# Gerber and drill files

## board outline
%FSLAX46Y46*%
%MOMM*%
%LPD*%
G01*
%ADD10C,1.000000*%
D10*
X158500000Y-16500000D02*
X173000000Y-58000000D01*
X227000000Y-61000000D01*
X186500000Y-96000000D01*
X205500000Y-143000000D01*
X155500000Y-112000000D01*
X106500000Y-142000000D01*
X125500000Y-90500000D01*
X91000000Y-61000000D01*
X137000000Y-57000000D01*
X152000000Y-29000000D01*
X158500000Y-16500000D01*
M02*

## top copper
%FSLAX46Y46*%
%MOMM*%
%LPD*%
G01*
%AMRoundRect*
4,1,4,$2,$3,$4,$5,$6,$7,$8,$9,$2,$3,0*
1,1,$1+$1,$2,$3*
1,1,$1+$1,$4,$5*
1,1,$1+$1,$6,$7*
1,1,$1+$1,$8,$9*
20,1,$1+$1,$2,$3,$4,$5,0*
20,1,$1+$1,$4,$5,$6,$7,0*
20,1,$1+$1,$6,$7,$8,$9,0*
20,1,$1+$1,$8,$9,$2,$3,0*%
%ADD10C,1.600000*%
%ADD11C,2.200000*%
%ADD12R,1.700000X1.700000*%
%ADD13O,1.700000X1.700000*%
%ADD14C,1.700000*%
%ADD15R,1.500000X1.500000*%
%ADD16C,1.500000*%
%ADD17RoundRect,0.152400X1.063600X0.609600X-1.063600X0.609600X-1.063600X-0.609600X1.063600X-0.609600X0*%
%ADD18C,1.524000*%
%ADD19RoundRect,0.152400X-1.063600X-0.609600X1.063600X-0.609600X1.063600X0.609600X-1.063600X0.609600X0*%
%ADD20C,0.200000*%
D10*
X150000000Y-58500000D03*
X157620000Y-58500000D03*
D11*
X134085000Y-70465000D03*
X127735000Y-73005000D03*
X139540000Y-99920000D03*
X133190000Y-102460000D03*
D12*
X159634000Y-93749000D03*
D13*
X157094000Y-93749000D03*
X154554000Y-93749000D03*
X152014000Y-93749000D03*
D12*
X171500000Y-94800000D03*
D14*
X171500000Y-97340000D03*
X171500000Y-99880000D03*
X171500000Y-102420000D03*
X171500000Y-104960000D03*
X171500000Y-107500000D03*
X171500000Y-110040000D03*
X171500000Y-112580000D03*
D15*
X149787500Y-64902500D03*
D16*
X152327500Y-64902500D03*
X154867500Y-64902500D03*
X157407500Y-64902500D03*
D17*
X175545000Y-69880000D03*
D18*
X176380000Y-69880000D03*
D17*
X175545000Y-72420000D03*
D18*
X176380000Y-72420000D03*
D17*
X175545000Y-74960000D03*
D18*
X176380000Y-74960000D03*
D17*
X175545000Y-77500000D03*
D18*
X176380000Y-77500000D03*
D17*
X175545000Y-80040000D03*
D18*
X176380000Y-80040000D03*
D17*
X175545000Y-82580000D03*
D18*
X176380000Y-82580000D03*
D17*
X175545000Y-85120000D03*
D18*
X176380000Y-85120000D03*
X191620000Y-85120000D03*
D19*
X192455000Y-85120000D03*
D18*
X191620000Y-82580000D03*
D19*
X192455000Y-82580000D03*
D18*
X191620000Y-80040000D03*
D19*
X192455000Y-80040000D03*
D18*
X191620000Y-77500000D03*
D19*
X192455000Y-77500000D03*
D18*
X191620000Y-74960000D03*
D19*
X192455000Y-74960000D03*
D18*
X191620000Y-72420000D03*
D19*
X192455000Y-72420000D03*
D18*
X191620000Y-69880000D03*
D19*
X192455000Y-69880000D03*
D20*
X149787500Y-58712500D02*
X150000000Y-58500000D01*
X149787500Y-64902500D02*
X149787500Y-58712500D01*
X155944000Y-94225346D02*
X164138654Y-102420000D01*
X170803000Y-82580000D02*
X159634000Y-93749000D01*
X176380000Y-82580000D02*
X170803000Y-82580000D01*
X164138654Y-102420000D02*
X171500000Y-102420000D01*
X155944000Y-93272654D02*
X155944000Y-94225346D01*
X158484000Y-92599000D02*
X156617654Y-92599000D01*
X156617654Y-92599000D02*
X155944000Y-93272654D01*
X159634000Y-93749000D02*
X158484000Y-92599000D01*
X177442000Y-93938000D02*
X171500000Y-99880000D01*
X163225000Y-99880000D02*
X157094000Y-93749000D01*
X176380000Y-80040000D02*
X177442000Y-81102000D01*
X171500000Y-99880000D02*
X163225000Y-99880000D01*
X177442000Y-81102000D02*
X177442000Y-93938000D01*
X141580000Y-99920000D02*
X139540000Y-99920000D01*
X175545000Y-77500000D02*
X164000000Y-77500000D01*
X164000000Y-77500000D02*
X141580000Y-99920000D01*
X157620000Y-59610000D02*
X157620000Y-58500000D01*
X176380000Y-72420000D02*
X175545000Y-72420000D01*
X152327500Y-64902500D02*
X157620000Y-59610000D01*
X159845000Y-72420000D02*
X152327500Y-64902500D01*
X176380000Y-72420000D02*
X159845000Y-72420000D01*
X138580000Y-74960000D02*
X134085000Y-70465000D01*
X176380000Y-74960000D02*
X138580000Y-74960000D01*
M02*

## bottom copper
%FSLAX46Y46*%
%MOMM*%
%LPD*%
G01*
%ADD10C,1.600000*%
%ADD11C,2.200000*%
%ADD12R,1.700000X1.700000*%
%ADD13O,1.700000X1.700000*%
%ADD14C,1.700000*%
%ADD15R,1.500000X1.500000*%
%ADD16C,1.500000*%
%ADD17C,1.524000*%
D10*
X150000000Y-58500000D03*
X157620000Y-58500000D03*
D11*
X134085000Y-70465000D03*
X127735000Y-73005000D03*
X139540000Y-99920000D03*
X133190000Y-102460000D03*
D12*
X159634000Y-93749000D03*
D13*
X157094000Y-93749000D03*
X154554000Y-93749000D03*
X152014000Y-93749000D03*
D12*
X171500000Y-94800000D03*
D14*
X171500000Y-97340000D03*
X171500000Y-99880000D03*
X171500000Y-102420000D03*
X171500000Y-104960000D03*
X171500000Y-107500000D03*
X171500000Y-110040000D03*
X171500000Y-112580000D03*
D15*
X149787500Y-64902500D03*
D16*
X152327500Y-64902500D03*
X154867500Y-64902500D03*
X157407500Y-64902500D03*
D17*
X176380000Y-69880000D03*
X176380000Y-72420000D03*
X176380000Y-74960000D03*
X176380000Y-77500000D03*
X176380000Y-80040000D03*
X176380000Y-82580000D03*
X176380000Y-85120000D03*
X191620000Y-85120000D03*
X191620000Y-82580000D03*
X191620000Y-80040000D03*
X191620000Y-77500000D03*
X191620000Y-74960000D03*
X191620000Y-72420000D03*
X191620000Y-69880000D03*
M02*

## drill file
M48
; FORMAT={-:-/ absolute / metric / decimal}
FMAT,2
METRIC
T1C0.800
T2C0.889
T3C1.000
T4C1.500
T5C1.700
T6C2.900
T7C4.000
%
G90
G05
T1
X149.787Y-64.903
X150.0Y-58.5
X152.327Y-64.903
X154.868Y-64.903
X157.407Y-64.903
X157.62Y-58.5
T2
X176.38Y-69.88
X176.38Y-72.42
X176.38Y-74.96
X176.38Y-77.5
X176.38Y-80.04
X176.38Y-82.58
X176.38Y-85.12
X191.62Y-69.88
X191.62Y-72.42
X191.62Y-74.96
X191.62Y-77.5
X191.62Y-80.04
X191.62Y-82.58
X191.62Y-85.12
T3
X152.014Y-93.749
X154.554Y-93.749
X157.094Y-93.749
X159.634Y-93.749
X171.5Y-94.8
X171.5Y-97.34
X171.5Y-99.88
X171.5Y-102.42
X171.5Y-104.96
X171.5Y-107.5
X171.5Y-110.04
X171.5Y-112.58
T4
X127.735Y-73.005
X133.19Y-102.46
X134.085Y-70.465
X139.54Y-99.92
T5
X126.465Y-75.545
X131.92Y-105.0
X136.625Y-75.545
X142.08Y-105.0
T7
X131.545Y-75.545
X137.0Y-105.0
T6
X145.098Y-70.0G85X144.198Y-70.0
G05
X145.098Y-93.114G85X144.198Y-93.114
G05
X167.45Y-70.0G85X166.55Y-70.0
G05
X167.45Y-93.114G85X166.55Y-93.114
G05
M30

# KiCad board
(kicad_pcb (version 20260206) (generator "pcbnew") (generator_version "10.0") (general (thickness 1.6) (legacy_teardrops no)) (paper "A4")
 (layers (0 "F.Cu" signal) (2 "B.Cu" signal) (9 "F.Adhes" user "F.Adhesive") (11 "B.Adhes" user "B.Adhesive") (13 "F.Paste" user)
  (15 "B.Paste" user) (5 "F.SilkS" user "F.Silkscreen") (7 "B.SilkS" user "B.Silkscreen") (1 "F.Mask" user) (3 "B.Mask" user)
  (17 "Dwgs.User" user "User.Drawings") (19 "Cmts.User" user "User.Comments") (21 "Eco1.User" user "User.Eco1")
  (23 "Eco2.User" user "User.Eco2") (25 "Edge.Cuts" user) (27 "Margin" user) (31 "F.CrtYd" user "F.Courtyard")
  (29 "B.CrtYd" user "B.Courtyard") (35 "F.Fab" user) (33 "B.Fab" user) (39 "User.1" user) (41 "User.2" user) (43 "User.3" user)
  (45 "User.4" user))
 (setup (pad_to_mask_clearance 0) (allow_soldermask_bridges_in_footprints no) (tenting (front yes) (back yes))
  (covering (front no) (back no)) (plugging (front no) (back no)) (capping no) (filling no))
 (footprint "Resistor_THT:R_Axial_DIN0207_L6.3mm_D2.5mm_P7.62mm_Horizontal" (layer "F.Cu") (at 150 58.5)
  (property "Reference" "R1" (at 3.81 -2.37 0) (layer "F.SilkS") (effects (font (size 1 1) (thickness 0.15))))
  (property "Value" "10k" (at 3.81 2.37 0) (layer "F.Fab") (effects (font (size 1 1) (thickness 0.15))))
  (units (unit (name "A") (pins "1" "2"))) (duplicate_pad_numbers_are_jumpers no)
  (pad "1" thru_hole circle (at 0 0) (size 1.6 1.6) (drill 0.8) (layers "*.Cu" "*.Mask") (remove_unused_layers no) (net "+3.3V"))
  (pad "2" thru_hole circle (at 7.62 0) (size 1.6 1.6) (drill 0.8) (layers "*.Cu" "*.Mask") (remove_unused_layers no) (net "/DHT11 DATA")))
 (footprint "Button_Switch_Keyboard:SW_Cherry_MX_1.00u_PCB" (layer "F.Cu") (at 134.085 70.465)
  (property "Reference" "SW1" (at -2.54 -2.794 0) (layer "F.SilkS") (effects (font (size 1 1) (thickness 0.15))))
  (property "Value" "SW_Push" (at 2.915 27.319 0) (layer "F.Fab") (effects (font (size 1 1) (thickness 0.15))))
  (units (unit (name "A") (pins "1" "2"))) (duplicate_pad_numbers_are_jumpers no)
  (pad "" np_thru_hole circle (at -7.62 5.08) (size 1.7 1.7) (drill 1.7) (layers "*.Cu" "*.Mask"))
  (pad "" np_thru_hole circle (at -2.54 5.08) (size 4 4) (drill 4) (layers "*.Cu" "*.Mask"))
  (pad "" np_thru_hole circle (at 2.54 5.08) (size 1.7 1.7) (drill 1.7) (layers "*.Cu" "*.Mask"))
  (pad "1" thru_hole circle (at 0 0) (size 2.2 2.2) (drill 1.5) (layers "*.Cu" "*.Mask") (remove_unused_layers no) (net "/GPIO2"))
  (pad "2" thru_hole circle (at -6.35 2.54) (size 2.2 2.2) (drill 1.5) (layers "*.Cu" "*.Mask") (remove_unused_layers no) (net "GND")))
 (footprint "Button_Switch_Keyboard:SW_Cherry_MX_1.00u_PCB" (layer "F.Cu") (at 139.54 99.92)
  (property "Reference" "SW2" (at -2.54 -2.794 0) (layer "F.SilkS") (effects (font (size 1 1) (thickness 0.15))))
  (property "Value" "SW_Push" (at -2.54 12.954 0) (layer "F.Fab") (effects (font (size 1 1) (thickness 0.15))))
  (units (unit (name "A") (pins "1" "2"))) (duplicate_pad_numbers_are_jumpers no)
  (pad "" np_thru_hole circle (at -7.62 5.08) (size 1.7 1.7) (drill 1.7) (layers "*.Cu" "*.Mask"))
  (pad "" np_thru_hole circle (at -2.54 5.08) (size 4 4) (drill 4) (layers "*.Cu" "*.Mask"))
  (pad "" np_thru_hole circle (at 2.54 5.08) (size 1.7 1.7) (drill 1.7) (layers "*.Cu" "*.Mask"))
  (pad "1" thru_hole circle (at 0 0) (size 2.2 2.2) (drill 1.5) (layers "*.Cu" "*.Mask") (remove_unused_layers no) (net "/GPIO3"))
  (pad "2" thru_hole circle (at -6.35 2.54) (size 2.2 2.2) (drill 1.5) (layers "*.Cu" "*.Mask") (remove_unused_layers no) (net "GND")))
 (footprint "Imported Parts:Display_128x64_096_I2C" (layer "F.Cu") (at 155.824 93.749 180)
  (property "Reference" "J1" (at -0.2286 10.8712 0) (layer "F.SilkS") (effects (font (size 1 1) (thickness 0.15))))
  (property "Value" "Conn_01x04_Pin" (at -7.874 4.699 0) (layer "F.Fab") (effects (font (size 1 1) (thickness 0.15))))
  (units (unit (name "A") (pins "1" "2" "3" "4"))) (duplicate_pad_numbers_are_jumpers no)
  (pad "" np_thru_hole oval (at -11.176 0.635 180) (size 3.8 2.9) (drill oval 3.8 2.9) (layers "*.Cu" "*.Mask"))
  (pad "" np_thru_hole oval (at -11.176 23.749 180) (size 3.8 2.9) (drill oval 3.8 2.9) (layers "*.Cu" "*.Mask"))
  (pad "" np_thru_hole oval (at 11.176 0.635 180) (size 3.8 2.9) (drill oval 3.8 2.9) (layers "*.Cu" "*.Mask"))
  (pad "" np_thru_hole oval (at 11.176 23.749 180) (size 3.8 2.9) (drill oval 3.8 2.9) (layers "*.Cu" "*.Mask"))
  (pad "1" thru_hole rect (at -3.81 0 270) (size 1.7 1.7) (drill 1) (layers "*.Cu" "*.Mask") (remove_unused_layers no) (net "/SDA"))
  (pad "2" thru_hole oval (at -1.27 0 270) (size 1.7 1.7) (drill 1) (layers "*.Cu" "*.Mask") (remove_unused_layers no) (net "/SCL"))
  (pad "3" thru_hole oval (at 1.27 0 270) (size 1.7 1.7) (drill 1) (layers "*.Cu" "*.Mask") (remove_unused_layers no) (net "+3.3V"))
  (pad "4" thru_hole oval (at 3.81 0 270) (size 1.7 1.7) (drill 1) (layers "*.Cu" "*.Mask") (remove_unused_layers no) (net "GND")))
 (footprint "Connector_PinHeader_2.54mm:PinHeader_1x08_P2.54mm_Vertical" (layer "F.Cu") (at 171.5 94.8)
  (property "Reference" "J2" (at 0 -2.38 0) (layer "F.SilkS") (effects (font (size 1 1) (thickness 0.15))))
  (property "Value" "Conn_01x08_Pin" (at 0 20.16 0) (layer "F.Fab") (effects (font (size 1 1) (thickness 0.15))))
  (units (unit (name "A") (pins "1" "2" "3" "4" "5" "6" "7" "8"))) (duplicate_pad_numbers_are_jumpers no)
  (pad "1" thru_hole rect (at 0 0) (size 1.7 1.7) (drill 1) (layers "*.Cu" "*.Mask") (remove_unused_layers no) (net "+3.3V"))
  (pad "2" thru_hole circle (at 0 2.54) (size 1.7 1.7) (drill 1) (layers "*.Cu" "*.Mask") (remove_unused_layers no) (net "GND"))
  (pad "3" thru_hole circle (at 0 5.08) (size 1.7 1.7) (drill 1) (layers "*.Cu" "*.Mask") (remove_unused_layers no) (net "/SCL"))
  (pad "4" thru_hole circle (at 0 7.62) (size 1.7 1.7) (drill 1) (layers "*.Cu" "*.Mask") (remove_unused_layers no) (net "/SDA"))
  (pad "5" thru_hole circle (at 0 10.16) (size 1.7 1.7) (drill 1) (layers "*.Cu" "*.Mask") (remove_unused_layers no)
   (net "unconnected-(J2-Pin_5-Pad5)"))
  (pad "6" thru_hole circle (at 0 12.7) (size 1.7 1.7) (drill 1) (layers "*.Cu" "*.Mask") (remove_unused_layers no)
   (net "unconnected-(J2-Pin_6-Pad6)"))
  (pad "7" thru_hole circle (at 0 15.24) (size 1.7 1.7) (drill 1) (layers "*.Cu" "*.Mask") (remove_unused_layers no)
   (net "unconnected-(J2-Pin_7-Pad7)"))
  (pad "8" thru_hole circle (at 0 17.78) (size 1.7 1.7) (drill 1) (layers "*.Cu" "*.Mask") (remove_unused_layers no)
   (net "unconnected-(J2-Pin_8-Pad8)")))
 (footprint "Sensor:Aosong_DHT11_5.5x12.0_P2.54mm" (layer "F.Cu") (at 149.7875 64.9025 90)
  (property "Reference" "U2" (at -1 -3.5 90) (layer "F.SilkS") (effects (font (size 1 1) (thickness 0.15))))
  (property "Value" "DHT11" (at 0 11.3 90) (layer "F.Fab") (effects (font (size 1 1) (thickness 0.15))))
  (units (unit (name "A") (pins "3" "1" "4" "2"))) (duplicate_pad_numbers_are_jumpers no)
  (pad "1" thru_hole rect (at 0 0 90) (size 1.5 1.5) (drill 0.8) (layers "*.Cu" "*.Mask") (remove_unused_layers no) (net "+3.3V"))
  (pad "2" thru_hole circle (at 0 2.54 90) (size 1.5 1.5) (drill 0.8) (layers "*.Cu" "*.Mask") (remove_unused_layers no) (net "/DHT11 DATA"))
  (pad "3" thru_hole circle (at 0 5.08 90) (size 1.5 1.5) (drill 0.8) (layers "*.Cu" "*.Mask") (remove_unused_layers no)
   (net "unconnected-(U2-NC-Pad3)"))
  (pad "4" thru_hole circle (at 0 7.62 90) (size 1.5 1.5) (drill 0.8) (layers "*.Cu" "*.Mask") (remove_unused_layers no) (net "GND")))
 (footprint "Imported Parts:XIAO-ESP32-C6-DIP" (layer "F.Cu") (at 184 77.5 90)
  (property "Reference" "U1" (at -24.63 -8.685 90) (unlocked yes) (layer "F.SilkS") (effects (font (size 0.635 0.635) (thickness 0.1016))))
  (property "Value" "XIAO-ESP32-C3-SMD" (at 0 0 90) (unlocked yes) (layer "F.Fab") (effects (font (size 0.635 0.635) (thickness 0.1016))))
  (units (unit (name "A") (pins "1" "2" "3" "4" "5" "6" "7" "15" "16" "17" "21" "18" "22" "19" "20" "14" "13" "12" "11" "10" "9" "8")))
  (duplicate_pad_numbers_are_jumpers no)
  (pad "1" smd roundrect (at 7.62 -8.455 180) (size 2.432 1.524) (layers "F.Cu" "F.Mask") (roundrect_rratio 0.1)
   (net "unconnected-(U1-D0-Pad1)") (thermal_bridge_angle 45))
  (pad "1" thru_hole circle (at 7.62 -7.62 180) (size 1.524 1.524) (drill 0.889) (layers "*.Cu" "*.Mask") (remove_unused_layers no)
   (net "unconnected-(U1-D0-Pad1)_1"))
  (pad "2" smd roundrect (at 5.08 -8.455 180) (size 2.432 1.524) (layers "F.Cu" "F.Mask") (roundrect_rratio 0.1) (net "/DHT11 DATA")
   (thermal_bridge_angle 45))
  (pad "2" thru_hole circle (at 5.08 -7.62 180) (size 1.524 1.524) (drill 0.889) (layers "*.Cu" "*.Mask") (remove_unused_layers no)
   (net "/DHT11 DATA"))
  (pad "3" smd roundrect (at 2.54 -8.455 180) (size 2.432 1.524) (layers "F.Cu" "F.Mask") (roundrect_rratio 0.1) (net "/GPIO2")
   (thermal_bridge_angle 45))
  (pad "3" thru_hole circle (at 2.54 -7.62 180) (size 1.524 1.524) (drill 0.889) (layers "*.Cu" "*.Mask") (remove_unused_layers no)
   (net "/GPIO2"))
  (pad "4" smd roundrect (at 0 -8.455 180) (size 2.432 1.524) (layers "F.Cu" "F.Mask") (roundrect_rratio 0.1) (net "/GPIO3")
   (thermal_bridge_angle 45))
  (pad "4" thru_hole circle (at 0 -7.62 180) (size 1.524 1.524) (drill 0.889) (layers "*.Cu" "*.Mask") (remove_unused_layers no)
   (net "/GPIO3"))
  (pad "5" smd roundrect (at -2.54 -8.455 180) (size 2.432 1.524) (layers "F.Cu" "F.Mask") (roundrect_rratio 0.1) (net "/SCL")
   (thermal_bridge_angle 45))
  (pad "5" thru_hole circle (at -2.54 -7.62 180) (size 1.524 1.524) (drill 0.889) (layers "*.Cu" "*.Mask") (remove_unused_layers no)
   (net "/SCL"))
  (pad "6" smd roundrect (at -5.08 -8.455 180) (size 2.432 1.524) (layers "F.Cu" "F.Mask") (roundrect_rratio 0.1) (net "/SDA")
   (thermal_bridge_angle 45))
  (pad "6" thru_hole circle (at -5.08 -7.62 180) (size 1.524 1.524) (drill 0.889) (layers "*.Cu" "*.Mask") (remove_unused_layers no)
   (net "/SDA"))
  (pad "7" smd roundrect (at -7.62 -8.455 180) (size 2.432 1.524) (layers "F.Cu" "F.Mask") (roundrect_rratio 0.1)
   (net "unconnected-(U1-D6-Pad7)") (thermal_bridge_angle 45))
  (pad "7" thru_hole circle (at -7.62 -7.62 180) (size 1.524 1.524) (drill 0.889) (layers "*.Cu" "*.Mask") (remove_unused_layers no)
   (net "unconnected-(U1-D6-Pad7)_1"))
  (pad "8" thru_hole circle (at -7.62 7.62) (size 1.524 1.524) (drill 0.889) (layers "*.Cu" "*.Mask") (remove_unused_layers no)
   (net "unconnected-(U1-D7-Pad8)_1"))
  (pad "8" smd roundrect (at -7.62 8.455) (size 2.432 1.524) (layers "F.Cu" "F.Mask") (roundrect_rratio 0.1)
   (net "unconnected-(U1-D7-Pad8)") (thermal_bridge_angle 45))
  (pad "9" thru_hole circle (at -5.08 7.62) (size 1.524 1.524) (drill 0.889) (layers "*.Cu" "*.Mask") (remove_unused_layers no)
   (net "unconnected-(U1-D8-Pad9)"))
  (pad "9" smd roundrect (at -5.08 8.455) (size 2.432 1.524) (layers "F.Cu" "F.Mask") (roundrect_rratio 0.1)
   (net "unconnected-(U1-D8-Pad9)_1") (thermal_bridge_angle 45))
  (pad "10" thru_hole circle (at -2.54 7.62) (size 1.524 1.524) (drill 0.889) (layers "*.Cu" "*.Mask") (remove_unused_layers no)
   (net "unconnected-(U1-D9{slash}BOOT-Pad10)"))
  (pad "10" smd roundrect (at -2.54 8.455) (size 2.432 1.524) (layers "F.Cu" "F.Mask") (roundrect_rratio 0.1)
   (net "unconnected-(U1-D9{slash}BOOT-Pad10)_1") (thermal_bridge_angle 45))
  (pad "11" thru_hole circle (at 0 7.62) (size 1.524 1.524) (drill 0.889) (layers "*.Cu" "*.Mask") (remove_unused_layers no)
   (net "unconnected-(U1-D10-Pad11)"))
  (pad "11" smd roundrect (at 0 8.455) (size 2.432 1.524) (layers "F.Cu" "F.Mask") (roundrect_rratio 0.1)
   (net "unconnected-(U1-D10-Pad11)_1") (thermal_bridge_angle 45))
  (pad "12" thru_hole circle (at 2.54 7.62) (size 1.524 1.524) (drill 0.889) (layers "*.Cu" "*.Mask") (remove_unused_layers no)
   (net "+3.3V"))
  (pad "12" smd roundrect (at 2.54 8.455) (size 2.432 1.524) (layers "F.Cu" "F.Mask") (roundrect_rratio 0.1) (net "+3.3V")
   (thermal_bridge_angle 45))
  (pad "13" thru_hole circle (at 5.08 7.62) (size 1.524 1.524) (drill 0.889) (layers "*.Cu" "*.Mask") (remove_unused_layers no) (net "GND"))
  (pad "13" smd roundrect (at 5.08 8.455) (size 2.432 1.524) (layers "F.Cu" "F.Mask") (roundrect_rratio 0.1) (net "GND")
   (thermal_bridge_angle 45))
  (pad "14" thru_hole circle (at 7.62 7.62) (size 1.524 1.524) (drill 0.889) (layers "*.Cu" "*.Mask") (remove_unused_layers no) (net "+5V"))
  (pad "14" smd roundrect (at 7.62 8.455) (size 2.432 1.524) (layers "F.Cu" "F.Mask") (roundrect_rratio 0.1) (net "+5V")
   (thermal_bridge_angle 45)))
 (gr_poly
  (pts (xy 158.5 16.5) (xy 173 58) (xy 227 61) (xy 186.5 96) (xy 205.5 143) (xy 155.5 112) (xy 106.5 142) (xy 125.5 90.5) (xy 91 61)
   (xy 137 57) (xy 152 29))
  (stroke (width 1) (type solid)) (fill no) (layer "Edge.Cuts"))
 (segment (start 149.7875 58.7125) (end 150 58.5) (width 0.2) (layer "F.Cu") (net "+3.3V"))
 (segment (start 149.7875 64.9025) (end 149.7875 58.7125) (width 0.2) (layer "F.Cu") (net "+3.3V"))
 (segment (start 155.944 94.225346) (end 164.138654 102.42) (width 0.2) (layer "F.Cu") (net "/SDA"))
 (segment (start 170.803 82.58) (end 159.634 93.749) (width 0.2) (layer "F.Cu") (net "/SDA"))
 (segment (start 176.38 82.58) (end 170.803 82.58) (width 0.2) (layer "F.Cu") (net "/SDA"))
 (segment (start 164.138654 102.42) (end 171.5 102.42) (width 0.2) (layer "F.Cu") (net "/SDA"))
 (segment (start 155.944 93.272654) (end 155.944 94.225346) (width 0.2) (layer "F.Cu") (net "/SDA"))
 (segment (start 158.484 92.599) (end 156.617654 92.599) (width 0.2) (layer "F.Cu") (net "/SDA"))
 (segment (start 156.617654 92.599) (end 155.944 93.272654) (width 0.2) (layer "F.Cu") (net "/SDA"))
 (segment (start 159.634 93.749) (end 158.484 92.599) (width 0.2) (layer "F.Cu") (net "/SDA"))
 (segment (start 177.442 93.938) (end 171.5 99.88) (width 0.2) (layer "F.Cu") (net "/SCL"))
 (segment (start 163.225 99.88) (end 157.094 93.749) (width 0.2) (layer "F.Cu") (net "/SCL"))
 (segment (start 176.38 80.04) (end 177.442 81.102) (width 0.2) (layer "F.Cu") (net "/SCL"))
 (segment (start 171.5 99.88) (end 163.225 99.88) (width 0.2) (layer "F.Cu") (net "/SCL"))
 (segment (start 177.442 81.102) (end 177.442 93.938) (width 0.2) (layer "F.Cu") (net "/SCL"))
 (segment (start 141.58 99.92) (end 139.54 99.92) (width 0.2) (layer "F.Cu") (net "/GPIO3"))
 (segment (start 175.545 77.5) (end 164 77.5) (width 0.2) (layer "F.Cu") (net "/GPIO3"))
 (segment (start 164 77.5) (end 141.58 99.92) (width 0.2) (layer "F.Cu") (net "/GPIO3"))
 (segment (start 157.62 59.61) (end 157.62 58.5) (width 0.2) (layer "F.Cu") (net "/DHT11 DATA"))
 (segment (start 176.38 72.42) (end 175.545 72.42) (width 0.2) (layer "F.Cu") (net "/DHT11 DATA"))
 (segment (start 152.3275 64.9025) (end 157.62 59.61) (width 0.2) (layer "F.Cu") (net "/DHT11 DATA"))
 (segment (start 159.845 72.42) (end 152.3275 64.9025) (width 0.2) (layer "F.Cu") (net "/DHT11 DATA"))
 (segment (start 176.38 72.42) (end 159.845 72.42) (width 0.2) (layer "F.Cu") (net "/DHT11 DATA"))
 (segment (start 138.58 74.96) (end 134.085 70.465) (width 0.2) (layer "F.Cu") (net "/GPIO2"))
 (segment (start 176.38 74.96) (end 138.58 74.96) (width 0.2) (layer "F.Cu") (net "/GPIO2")))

